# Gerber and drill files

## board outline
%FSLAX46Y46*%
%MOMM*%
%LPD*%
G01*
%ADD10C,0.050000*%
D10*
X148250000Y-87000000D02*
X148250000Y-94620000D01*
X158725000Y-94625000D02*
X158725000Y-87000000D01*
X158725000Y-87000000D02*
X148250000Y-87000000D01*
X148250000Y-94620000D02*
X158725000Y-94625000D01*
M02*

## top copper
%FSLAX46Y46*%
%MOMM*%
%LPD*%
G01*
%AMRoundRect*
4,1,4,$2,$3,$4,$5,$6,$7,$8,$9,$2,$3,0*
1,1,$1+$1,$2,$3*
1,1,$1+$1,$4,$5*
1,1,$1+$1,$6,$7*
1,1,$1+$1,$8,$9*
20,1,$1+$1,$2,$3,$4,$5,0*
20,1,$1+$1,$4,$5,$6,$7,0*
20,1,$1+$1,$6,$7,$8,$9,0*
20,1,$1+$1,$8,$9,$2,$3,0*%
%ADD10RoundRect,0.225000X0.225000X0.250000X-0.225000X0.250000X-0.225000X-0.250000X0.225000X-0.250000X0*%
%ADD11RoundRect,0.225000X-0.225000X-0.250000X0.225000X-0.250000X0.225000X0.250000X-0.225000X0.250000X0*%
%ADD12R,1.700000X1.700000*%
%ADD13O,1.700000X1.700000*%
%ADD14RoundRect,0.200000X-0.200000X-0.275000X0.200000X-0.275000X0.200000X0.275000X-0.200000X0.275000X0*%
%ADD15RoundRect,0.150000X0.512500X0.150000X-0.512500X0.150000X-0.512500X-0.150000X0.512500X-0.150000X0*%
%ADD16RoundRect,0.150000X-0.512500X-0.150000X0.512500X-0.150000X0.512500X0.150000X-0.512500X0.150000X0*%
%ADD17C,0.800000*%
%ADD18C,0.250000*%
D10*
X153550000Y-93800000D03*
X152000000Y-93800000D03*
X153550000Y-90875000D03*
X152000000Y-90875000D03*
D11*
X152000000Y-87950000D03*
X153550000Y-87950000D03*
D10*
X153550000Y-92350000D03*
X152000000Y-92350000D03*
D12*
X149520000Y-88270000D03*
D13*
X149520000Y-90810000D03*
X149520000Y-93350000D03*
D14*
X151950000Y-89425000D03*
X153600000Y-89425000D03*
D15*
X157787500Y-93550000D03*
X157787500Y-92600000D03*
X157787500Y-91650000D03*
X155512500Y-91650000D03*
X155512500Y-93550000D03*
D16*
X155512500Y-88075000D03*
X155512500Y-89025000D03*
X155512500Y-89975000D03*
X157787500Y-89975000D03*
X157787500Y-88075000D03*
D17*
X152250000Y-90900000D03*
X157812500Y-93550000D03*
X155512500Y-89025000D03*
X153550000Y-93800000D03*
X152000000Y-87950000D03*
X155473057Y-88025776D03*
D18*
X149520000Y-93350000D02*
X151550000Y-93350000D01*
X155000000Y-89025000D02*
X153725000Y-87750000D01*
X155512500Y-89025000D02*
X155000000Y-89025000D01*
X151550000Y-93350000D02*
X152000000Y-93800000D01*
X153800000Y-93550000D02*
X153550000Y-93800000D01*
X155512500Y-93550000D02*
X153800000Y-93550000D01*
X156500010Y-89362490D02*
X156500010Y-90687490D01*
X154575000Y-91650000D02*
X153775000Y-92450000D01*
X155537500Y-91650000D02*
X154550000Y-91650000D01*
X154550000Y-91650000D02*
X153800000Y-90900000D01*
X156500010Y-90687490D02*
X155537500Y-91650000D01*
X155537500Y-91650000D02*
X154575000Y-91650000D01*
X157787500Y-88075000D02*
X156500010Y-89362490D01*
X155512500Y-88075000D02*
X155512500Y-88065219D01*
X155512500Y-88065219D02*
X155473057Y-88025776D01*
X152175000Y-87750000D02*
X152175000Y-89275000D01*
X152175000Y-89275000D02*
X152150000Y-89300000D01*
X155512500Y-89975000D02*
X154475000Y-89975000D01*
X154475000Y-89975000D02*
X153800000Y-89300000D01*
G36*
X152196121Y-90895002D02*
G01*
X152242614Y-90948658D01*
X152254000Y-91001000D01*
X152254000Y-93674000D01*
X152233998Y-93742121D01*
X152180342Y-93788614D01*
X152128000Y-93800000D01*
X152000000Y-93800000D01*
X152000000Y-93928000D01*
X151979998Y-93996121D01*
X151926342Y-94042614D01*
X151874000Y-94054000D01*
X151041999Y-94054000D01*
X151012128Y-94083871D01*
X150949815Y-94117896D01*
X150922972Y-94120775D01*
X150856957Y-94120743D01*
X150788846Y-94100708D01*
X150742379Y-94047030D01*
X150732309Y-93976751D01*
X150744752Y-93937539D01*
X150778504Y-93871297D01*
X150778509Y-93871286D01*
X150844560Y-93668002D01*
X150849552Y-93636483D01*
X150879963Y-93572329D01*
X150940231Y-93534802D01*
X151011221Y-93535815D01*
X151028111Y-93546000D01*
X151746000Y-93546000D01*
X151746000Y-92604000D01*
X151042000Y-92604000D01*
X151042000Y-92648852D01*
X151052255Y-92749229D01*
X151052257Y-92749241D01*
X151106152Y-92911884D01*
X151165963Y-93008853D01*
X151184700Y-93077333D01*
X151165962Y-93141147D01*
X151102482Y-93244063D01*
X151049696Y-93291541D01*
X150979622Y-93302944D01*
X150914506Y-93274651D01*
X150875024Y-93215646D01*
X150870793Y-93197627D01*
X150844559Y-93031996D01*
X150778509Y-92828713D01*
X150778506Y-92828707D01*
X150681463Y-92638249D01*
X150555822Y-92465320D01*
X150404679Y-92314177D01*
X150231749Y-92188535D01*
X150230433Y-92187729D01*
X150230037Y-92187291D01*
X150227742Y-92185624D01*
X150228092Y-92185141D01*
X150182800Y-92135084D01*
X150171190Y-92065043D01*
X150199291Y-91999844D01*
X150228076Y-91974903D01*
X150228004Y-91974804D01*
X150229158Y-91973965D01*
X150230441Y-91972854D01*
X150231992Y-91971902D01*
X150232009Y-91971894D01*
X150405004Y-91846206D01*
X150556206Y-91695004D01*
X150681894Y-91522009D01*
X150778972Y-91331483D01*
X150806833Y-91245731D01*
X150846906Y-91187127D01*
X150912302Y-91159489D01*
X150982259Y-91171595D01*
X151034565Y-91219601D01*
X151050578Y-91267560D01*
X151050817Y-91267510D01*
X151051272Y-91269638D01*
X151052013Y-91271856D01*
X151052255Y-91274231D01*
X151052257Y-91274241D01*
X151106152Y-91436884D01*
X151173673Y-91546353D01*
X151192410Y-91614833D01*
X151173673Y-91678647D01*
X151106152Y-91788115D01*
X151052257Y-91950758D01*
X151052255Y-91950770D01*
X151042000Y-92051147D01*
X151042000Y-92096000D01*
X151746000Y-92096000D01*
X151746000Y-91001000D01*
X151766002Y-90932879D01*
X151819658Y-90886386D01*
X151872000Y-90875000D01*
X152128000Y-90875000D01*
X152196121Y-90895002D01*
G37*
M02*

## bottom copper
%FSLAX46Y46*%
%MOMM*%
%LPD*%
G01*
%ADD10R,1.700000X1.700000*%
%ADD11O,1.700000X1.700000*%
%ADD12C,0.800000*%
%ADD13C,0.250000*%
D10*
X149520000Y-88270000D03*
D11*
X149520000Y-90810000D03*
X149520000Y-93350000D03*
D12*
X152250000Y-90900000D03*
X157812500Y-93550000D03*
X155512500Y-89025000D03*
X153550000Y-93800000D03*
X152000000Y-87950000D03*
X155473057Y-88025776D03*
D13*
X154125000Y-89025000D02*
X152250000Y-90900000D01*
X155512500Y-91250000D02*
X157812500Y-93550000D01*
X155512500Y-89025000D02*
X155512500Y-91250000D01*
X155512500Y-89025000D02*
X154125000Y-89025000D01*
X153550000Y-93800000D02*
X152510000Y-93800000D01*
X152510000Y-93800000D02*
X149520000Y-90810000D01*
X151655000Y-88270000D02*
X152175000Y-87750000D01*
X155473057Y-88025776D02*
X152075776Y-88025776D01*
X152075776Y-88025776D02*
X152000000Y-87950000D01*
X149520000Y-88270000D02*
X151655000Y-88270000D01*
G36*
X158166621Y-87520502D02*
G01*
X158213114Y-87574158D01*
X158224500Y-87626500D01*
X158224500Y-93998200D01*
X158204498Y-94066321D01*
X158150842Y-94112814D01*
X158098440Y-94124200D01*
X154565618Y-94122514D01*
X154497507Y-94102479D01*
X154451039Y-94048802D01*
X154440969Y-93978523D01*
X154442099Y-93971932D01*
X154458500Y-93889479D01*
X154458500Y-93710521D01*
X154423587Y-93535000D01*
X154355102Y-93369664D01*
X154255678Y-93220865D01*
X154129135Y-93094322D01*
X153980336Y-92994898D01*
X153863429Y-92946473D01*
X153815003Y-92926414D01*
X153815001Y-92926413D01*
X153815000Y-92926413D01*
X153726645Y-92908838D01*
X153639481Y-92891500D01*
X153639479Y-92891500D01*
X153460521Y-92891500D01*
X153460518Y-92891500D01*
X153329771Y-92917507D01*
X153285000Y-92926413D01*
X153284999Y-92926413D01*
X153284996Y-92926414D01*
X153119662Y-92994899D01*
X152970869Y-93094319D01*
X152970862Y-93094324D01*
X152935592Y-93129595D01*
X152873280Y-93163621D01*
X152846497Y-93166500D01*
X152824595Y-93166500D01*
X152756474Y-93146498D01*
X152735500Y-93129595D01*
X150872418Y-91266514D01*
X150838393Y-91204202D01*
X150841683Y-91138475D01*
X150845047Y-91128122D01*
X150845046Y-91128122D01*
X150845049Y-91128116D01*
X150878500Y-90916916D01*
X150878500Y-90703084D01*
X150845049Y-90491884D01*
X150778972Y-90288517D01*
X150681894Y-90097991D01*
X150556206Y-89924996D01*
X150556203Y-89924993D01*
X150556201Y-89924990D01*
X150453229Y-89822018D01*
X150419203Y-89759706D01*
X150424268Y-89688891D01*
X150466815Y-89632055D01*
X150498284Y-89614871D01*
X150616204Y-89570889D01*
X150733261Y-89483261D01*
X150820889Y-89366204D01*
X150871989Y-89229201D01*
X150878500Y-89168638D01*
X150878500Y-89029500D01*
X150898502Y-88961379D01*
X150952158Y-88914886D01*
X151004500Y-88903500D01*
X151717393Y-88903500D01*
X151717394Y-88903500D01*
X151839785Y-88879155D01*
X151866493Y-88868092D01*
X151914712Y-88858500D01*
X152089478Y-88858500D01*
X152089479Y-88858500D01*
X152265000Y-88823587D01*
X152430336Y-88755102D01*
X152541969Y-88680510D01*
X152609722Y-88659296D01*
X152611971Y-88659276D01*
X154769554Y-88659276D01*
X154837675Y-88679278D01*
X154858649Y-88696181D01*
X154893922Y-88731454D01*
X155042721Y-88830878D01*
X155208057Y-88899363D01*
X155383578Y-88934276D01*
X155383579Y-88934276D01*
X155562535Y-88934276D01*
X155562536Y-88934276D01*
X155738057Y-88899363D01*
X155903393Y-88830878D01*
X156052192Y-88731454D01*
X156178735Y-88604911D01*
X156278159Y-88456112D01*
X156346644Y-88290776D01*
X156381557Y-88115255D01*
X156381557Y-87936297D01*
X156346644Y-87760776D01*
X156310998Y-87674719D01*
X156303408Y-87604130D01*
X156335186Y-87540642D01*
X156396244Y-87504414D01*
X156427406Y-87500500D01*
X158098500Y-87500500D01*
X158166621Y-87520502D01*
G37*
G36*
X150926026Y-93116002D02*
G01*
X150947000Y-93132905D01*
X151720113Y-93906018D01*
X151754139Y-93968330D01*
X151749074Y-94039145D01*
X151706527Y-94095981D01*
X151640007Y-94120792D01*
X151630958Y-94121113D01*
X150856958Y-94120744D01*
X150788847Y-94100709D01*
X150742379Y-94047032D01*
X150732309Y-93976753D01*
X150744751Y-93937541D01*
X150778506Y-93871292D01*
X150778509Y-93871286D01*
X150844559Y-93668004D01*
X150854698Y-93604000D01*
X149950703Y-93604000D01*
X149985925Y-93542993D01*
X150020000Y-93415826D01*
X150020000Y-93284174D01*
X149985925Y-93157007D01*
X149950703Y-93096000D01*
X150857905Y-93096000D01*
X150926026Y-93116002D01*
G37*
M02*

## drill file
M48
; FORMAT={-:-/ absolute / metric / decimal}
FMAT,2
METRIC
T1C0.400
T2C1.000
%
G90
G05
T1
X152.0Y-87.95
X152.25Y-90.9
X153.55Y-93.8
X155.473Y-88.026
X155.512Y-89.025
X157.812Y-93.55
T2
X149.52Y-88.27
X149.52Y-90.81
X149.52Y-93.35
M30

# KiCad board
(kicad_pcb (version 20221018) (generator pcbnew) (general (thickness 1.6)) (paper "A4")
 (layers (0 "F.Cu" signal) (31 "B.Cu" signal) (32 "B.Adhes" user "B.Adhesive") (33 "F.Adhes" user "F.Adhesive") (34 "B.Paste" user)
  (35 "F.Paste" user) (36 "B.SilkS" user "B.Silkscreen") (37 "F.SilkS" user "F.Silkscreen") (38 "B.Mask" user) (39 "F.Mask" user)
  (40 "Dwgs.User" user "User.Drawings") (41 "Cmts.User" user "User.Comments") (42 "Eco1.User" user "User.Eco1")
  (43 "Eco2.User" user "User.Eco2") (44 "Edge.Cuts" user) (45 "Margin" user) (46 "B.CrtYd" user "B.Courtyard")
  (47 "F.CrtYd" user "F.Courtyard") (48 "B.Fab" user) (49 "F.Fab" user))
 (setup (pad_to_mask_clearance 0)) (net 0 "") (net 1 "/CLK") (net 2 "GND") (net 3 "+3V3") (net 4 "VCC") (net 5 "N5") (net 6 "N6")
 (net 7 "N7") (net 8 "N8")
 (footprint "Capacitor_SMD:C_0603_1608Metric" (layer "F.Cu") (at 152.775 93.8 180)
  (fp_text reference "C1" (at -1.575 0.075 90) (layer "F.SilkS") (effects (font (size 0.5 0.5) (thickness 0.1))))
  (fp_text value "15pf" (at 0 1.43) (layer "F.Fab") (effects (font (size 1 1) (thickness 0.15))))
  (pad "1" smd roundrect (at -0.775 0 180) (size 0.9 0.95) (layers "F.Cu" "F.Paste" "F.Mask") (roundrect_rratio 0.25) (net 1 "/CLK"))
  (pad "2" smd roundrect (at 0.775 0 180) (size 0.9 0.95) (layers "F.Cu" "F.Paste" "F.Mask") (roundrect_rratio 0.25) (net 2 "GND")))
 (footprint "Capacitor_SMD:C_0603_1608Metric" (layer "F.Cu") (at 152.775 90.875 180)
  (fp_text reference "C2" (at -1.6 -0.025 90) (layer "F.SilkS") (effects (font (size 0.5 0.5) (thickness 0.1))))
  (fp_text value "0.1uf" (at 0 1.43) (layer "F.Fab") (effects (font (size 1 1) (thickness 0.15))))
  (pad "1" smd roundrect (at -0.775 0 180) (size 0.9 0.95) (layers "F.Cu" "F.Paste" "F.Mask") (roundrect_rratio 0.25) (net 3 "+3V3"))
  (pad "2" smd roundrect (at 0.775 0 180) (size 0.9 0.95) (layers "F.Cu" "F.Paste" "F.Mask") (roundrect_rratio 0.25) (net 2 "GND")))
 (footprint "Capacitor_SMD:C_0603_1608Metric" (layer "F.Cu") (at 152.775 87.95)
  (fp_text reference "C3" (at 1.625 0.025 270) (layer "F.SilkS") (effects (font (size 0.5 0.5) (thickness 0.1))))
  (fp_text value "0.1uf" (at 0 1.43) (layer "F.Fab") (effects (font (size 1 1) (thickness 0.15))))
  (pad "1" smd roundrect (at -0.775 0) (size 0.9 0.95) (layers "F.Cu" "F.Paste" "F.Mask") (roundrect_rratio 0.25) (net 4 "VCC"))
  (pad "2" smd roundrect (at 0.775 0) (size 0.9 0.95) (layers "F.Cu" "F.Paste" "F.Mask") (roundrect_rratio 0.25) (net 2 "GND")))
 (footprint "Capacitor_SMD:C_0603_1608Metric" (layer "F.Cu") (at 152.775 92.35 180)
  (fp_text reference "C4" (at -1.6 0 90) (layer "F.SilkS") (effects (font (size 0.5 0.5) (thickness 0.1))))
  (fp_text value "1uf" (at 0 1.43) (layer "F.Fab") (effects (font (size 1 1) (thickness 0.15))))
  (pad "1" smd roundrect (at -0.775 0 180) (size 0.9 0.95) (layers "F.Cu" "F.Paste" "F.Mask") (roundrect_rratio 0.25) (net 3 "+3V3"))
  (pad "2" smd roundrect (at 0.775 0 180) (size 0.9 0.95) (layers "F.Cu" "F.Paste" "F.Mask") (roundrect_rratio 0.25) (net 2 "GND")))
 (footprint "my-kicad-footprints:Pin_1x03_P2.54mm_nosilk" (layer "F.Cu") (at 149.52 88.27)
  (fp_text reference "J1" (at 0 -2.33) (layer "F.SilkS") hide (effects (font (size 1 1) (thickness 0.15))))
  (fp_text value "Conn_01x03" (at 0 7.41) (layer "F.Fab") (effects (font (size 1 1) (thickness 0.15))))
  (pad "1" thru_hole rect (at 0 0) (size 1.7 1.7) (drill 1) (layers "*.Cu" "*.Mask") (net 4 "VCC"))
  (pad "2" thru_hole oval (at 0 2.54) (size 1.7 1.7) (drill 1) (layers "*.Cu" "*.Mask") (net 1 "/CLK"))
  (pad "3" thru_hole oval (at 0 5.08) (size 1.7 1.7) (drill 1) (layers "*.Cu" "*.Mask") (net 2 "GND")))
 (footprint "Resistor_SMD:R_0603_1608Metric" (layer "F.Cu") (at 152.775 89.425)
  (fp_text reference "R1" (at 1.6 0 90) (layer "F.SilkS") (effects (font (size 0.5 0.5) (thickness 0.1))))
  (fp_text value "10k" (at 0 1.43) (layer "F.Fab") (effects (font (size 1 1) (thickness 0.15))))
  (pad "1" smd roundrect (at -0.825 0) (size 0.8 0.95) (layers "F.Cu" "F.Paste" "F.Mask") (roundrect_rratio 0.25) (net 4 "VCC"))
  (pad "2" smd roundrect (at 0.825 0) (size 0.8 0.95) (layers "F.Cu" "F.Paste" "F.Mask") (roundrect_rratio 0.25) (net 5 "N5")))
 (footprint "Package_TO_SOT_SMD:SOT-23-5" (layer "F.Cu") (at 156.65 92.6 180)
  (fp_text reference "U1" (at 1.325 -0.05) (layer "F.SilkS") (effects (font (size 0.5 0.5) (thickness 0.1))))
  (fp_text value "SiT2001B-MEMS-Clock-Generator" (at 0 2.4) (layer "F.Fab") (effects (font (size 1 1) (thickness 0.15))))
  (pad "1" smd roundrect (at -1.1375 -0.95 180) (size 1.325 0.6) (layers "F.Cu" "F.Paste" "F.Mask") (roundrect_rratio 0.25) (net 2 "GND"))
  (pad "2" smd roundrect (at -1.1375 0 180) (size 1.325 0.6) (layers "F.Cu" "F.Paste" "F.Mask") (roundrect_rratio 0.25) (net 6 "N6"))
  (pad "3" smd roundrect (at -1.1375 0.95 180) (size 1.325 0.6) (layers "F.Cu" "F.Paste" "F.Mask") (roundrect_rratio 0.25) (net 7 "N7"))
  (pad "4" smd roundrect (at 1.1375 0.95 180) (size 1.325 0.6) (layers "F.Cu" "F.Paste" "F.Mask") (roundrect_rratio 0.25) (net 3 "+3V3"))
  (pad "5" smd roundrect (at 1.1375 -0.95 180) (size 1.325 0.6) (layers "F.Cu" "F.Paste" "F.Mask") (roundrect_rratio 0.25) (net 1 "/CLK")))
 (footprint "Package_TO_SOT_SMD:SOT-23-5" (layer "F.Cu") (at 156.65 89.025)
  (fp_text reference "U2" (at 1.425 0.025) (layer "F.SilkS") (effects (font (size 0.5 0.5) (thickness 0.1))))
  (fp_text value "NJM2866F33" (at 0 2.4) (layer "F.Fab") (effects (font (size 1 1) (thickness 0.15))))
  (pad "1" smd roundrect (at -1.1375 -0.95) (size 1.325 0.6) (layers "F.Cu" "F.Paste" "F.Mask") (roundrect_rratio 0.25) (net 4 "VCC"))
  (pad "2" smd roundrect (at -1.1375 0) (size 1.325 0.6) (layers "F.Cu" "F.Paste" "F.Mask") (roundrect_rratio 0.25) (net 2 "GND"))
  (pad "3" smd roundrect (at -1.1375 0.95) (size 1.325 0.6) (layers "F.Cu" "F.Paste" "F.Mask") (roundrect_rratio 0.25) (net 5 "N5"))
  (pad "4" smd roundrect (at 1.1375 0.95) (size 1.325 0.6) (layers "F.Cu" "F.Paste" "F.Mask") (roundrect_rratio 0.25) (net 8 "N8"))
  (pad "5" smd roundrect (at 1.1375 -0.95) (size 1.325 0.6) (layers "F.Cu" "F.Paste" "F.Mask") (roundrect_rratio 0.25) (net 3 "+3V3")))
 (gr_line (start 148.25 87) (end 148.25 94.62) (stroke (width 0.05) (type solid)) (layer "Edge.Cuts"))
 (gr_line (start 158.725 94.625) (end 158.725 87) (stroke (width 0.05) (type solid)) (layer "Edge.Cuts"))
 (gr_line (start 158.725 87) (end 148.25 87) (stroke (width 0.05) (type solid)) (layer "Edge.Cuts"))
 (gr_line (start 148.25 94.62) (end 158.725 94.625) (stroke (width 0.05) (type solid)) (layer "Edge.Cuts"))
 (segment (start 149.52 93.35) (end 151.55 93.35) (width 0.25) (layer "F.Cu") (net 2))
 (segment (start 155 89.025) (end 153.725 87.75) (width 0.25) (layer "F.Cu") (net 2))
 (segment (start 155.5125 89.025) (end 155 89.025) (width 0.25) (layer "F.Cu") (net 2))
 (segment (start 151.55 93.35) (end 152 93.8) (width 0.25) (layer "F.Cu") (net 2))
 (via (at 152.25 90.9) (size 0.8) (drill 0.4) (layers "F.Cu" "B.Cu") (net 2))
 (via (at 157.8125 93.55) (size 0.8) (drill 0.4) (layers "F.Cu" "B.Cu") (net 2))
 (via (at 155.5125 89.025) (size 0.8) (drill 0.4) (layers "F.Cu" "B.Cu") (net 2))
 (segment (start 154.125 89.025) (end 152.25 90.9) (width 0.25) (layer "B.Cu") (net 2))
 (segment (start 155.5125 91.25) (end 157.8125 93.55) (width 0.25) (layer "B.Cu") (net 2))
 (segment (start 155.5125 89.025) (end 155.5125 91.25) (width 0.25) (layer "B.Cu") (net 2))
 (segment (start 155.5125 89.025) (end 154.125 89.025) (width 0.25) (layer "B.Cu") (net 2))
 (segment (start 153.8 93.55) (end 153.55 93.8) (width 0.25) (layer "F.Cu") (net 1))
 (segment (start 155.5125 93.55) (end 153.8 93.55) (width 0.25) (layer "F.Cu") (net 1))
 (via (at 153.55 93.8) (size 0.8) (drill 0.4) (layers "F.Cu" "B.Cu") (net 1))
 (segment (start 153.55 93.8) (end 152.51 93.8) (width 0.25) (layer "B.Cu") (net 1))
 (segment (start 152.51 93.8) (end 149.52 90.81) (width 0.25) (layer "B.Cu") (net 1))
 (segment (start 156.50001 89.36249) (end 156.50001 90.68749) (width 0.25) (layer "F.Cu") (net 3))
 (segment (start 154.575 91.65) (end 153.775 92.45) (width 0.25) (layer "F.Cu") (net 3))
 (segment (start 155.5375 91.65) (end 154.55 91.65) (width 0.25) (layer "F.Cu") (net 3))
 (segment (start 154.55 91.65) (end 153.8 90.9) (width 0.25) (layer "F.Cu") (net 3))
 (segment (start 156.50001 90.68749) (end 155.5375 91.65) (width 0.25) (layer "F.Cu") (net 3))
 (segment (start 155.5375 91.65) (end 154.575 91.65) (width 0.25) (layer "F.Cu") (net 3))
 (segment (start 157.7875 88.075) (end 156.50001 89.36249) (width 0.25) (layer "F.Cu") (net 3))
 (segment (start 155.5125 88.075) (end 155.5125 88.065219) (width 0.25) (layer "F.Cu") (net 4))
 (segment (start 155.5125 88.065219) (end 155.473057 88.025776) (width 0.25) (layer "F.Cu") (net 4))
 (segment (start 152.175 87.75) (end 152.175 89.275) (width 0.25) (layer "F.Cu") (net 4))
 (segment (start 152.175 89.275) (end 152.15 89.3) (width 0.25) (layer "F.Cu") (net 4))
 (via (at 152 87.95) (size 0.8) (drill 0.4) (layers "F.Cu" "B.Cu") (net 4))
 (via (at 155.473057 88.025776) (size 0.8) (drill 0.4) (layers "F.Cu" "B.Cu") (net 4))
 (segment (start 151.655 88.27) (end 152.175 87.75) (width 0.25) (layer "B.Cu") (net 4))
 (segment (start 155.473057 88.025776) (end 152.075776 88.025776) (width 0.25) (layer "B.Cu") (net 4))
 (segment (start 152.075776 88.025776) (end 152 87.95) (width 0.25) (layer "B.Cu") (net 4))
 (segment (start 149.52 88.27) (end 151.655 88.27) (width 0.25) (layer "B.Cu") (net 4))
 (segment (start 155.5125 89.975) (end 154.475 89.975) (width 0.25) (layer "F.Cu") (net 5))
 (segment (start 154.475 89.975) (end 153.8 89.3) (width 0.25) (layer "F.Cu") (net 5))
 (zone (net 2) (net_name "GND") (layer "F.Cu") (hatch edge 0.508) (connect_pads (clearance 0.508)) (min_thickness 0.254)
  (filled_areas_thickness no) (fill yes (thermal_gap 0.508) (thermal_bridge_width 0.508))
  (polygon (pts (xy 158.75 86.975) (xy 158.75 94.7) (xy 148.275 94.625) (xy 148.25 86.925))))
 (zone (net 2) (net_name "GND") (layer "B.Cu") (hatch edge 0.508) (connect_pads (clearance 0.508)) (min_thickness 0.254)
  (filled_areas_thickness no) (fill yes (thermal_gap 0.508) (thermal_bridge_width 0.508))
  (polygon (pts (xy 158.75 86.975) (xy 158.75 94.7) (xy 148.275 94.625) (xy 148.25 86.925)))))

